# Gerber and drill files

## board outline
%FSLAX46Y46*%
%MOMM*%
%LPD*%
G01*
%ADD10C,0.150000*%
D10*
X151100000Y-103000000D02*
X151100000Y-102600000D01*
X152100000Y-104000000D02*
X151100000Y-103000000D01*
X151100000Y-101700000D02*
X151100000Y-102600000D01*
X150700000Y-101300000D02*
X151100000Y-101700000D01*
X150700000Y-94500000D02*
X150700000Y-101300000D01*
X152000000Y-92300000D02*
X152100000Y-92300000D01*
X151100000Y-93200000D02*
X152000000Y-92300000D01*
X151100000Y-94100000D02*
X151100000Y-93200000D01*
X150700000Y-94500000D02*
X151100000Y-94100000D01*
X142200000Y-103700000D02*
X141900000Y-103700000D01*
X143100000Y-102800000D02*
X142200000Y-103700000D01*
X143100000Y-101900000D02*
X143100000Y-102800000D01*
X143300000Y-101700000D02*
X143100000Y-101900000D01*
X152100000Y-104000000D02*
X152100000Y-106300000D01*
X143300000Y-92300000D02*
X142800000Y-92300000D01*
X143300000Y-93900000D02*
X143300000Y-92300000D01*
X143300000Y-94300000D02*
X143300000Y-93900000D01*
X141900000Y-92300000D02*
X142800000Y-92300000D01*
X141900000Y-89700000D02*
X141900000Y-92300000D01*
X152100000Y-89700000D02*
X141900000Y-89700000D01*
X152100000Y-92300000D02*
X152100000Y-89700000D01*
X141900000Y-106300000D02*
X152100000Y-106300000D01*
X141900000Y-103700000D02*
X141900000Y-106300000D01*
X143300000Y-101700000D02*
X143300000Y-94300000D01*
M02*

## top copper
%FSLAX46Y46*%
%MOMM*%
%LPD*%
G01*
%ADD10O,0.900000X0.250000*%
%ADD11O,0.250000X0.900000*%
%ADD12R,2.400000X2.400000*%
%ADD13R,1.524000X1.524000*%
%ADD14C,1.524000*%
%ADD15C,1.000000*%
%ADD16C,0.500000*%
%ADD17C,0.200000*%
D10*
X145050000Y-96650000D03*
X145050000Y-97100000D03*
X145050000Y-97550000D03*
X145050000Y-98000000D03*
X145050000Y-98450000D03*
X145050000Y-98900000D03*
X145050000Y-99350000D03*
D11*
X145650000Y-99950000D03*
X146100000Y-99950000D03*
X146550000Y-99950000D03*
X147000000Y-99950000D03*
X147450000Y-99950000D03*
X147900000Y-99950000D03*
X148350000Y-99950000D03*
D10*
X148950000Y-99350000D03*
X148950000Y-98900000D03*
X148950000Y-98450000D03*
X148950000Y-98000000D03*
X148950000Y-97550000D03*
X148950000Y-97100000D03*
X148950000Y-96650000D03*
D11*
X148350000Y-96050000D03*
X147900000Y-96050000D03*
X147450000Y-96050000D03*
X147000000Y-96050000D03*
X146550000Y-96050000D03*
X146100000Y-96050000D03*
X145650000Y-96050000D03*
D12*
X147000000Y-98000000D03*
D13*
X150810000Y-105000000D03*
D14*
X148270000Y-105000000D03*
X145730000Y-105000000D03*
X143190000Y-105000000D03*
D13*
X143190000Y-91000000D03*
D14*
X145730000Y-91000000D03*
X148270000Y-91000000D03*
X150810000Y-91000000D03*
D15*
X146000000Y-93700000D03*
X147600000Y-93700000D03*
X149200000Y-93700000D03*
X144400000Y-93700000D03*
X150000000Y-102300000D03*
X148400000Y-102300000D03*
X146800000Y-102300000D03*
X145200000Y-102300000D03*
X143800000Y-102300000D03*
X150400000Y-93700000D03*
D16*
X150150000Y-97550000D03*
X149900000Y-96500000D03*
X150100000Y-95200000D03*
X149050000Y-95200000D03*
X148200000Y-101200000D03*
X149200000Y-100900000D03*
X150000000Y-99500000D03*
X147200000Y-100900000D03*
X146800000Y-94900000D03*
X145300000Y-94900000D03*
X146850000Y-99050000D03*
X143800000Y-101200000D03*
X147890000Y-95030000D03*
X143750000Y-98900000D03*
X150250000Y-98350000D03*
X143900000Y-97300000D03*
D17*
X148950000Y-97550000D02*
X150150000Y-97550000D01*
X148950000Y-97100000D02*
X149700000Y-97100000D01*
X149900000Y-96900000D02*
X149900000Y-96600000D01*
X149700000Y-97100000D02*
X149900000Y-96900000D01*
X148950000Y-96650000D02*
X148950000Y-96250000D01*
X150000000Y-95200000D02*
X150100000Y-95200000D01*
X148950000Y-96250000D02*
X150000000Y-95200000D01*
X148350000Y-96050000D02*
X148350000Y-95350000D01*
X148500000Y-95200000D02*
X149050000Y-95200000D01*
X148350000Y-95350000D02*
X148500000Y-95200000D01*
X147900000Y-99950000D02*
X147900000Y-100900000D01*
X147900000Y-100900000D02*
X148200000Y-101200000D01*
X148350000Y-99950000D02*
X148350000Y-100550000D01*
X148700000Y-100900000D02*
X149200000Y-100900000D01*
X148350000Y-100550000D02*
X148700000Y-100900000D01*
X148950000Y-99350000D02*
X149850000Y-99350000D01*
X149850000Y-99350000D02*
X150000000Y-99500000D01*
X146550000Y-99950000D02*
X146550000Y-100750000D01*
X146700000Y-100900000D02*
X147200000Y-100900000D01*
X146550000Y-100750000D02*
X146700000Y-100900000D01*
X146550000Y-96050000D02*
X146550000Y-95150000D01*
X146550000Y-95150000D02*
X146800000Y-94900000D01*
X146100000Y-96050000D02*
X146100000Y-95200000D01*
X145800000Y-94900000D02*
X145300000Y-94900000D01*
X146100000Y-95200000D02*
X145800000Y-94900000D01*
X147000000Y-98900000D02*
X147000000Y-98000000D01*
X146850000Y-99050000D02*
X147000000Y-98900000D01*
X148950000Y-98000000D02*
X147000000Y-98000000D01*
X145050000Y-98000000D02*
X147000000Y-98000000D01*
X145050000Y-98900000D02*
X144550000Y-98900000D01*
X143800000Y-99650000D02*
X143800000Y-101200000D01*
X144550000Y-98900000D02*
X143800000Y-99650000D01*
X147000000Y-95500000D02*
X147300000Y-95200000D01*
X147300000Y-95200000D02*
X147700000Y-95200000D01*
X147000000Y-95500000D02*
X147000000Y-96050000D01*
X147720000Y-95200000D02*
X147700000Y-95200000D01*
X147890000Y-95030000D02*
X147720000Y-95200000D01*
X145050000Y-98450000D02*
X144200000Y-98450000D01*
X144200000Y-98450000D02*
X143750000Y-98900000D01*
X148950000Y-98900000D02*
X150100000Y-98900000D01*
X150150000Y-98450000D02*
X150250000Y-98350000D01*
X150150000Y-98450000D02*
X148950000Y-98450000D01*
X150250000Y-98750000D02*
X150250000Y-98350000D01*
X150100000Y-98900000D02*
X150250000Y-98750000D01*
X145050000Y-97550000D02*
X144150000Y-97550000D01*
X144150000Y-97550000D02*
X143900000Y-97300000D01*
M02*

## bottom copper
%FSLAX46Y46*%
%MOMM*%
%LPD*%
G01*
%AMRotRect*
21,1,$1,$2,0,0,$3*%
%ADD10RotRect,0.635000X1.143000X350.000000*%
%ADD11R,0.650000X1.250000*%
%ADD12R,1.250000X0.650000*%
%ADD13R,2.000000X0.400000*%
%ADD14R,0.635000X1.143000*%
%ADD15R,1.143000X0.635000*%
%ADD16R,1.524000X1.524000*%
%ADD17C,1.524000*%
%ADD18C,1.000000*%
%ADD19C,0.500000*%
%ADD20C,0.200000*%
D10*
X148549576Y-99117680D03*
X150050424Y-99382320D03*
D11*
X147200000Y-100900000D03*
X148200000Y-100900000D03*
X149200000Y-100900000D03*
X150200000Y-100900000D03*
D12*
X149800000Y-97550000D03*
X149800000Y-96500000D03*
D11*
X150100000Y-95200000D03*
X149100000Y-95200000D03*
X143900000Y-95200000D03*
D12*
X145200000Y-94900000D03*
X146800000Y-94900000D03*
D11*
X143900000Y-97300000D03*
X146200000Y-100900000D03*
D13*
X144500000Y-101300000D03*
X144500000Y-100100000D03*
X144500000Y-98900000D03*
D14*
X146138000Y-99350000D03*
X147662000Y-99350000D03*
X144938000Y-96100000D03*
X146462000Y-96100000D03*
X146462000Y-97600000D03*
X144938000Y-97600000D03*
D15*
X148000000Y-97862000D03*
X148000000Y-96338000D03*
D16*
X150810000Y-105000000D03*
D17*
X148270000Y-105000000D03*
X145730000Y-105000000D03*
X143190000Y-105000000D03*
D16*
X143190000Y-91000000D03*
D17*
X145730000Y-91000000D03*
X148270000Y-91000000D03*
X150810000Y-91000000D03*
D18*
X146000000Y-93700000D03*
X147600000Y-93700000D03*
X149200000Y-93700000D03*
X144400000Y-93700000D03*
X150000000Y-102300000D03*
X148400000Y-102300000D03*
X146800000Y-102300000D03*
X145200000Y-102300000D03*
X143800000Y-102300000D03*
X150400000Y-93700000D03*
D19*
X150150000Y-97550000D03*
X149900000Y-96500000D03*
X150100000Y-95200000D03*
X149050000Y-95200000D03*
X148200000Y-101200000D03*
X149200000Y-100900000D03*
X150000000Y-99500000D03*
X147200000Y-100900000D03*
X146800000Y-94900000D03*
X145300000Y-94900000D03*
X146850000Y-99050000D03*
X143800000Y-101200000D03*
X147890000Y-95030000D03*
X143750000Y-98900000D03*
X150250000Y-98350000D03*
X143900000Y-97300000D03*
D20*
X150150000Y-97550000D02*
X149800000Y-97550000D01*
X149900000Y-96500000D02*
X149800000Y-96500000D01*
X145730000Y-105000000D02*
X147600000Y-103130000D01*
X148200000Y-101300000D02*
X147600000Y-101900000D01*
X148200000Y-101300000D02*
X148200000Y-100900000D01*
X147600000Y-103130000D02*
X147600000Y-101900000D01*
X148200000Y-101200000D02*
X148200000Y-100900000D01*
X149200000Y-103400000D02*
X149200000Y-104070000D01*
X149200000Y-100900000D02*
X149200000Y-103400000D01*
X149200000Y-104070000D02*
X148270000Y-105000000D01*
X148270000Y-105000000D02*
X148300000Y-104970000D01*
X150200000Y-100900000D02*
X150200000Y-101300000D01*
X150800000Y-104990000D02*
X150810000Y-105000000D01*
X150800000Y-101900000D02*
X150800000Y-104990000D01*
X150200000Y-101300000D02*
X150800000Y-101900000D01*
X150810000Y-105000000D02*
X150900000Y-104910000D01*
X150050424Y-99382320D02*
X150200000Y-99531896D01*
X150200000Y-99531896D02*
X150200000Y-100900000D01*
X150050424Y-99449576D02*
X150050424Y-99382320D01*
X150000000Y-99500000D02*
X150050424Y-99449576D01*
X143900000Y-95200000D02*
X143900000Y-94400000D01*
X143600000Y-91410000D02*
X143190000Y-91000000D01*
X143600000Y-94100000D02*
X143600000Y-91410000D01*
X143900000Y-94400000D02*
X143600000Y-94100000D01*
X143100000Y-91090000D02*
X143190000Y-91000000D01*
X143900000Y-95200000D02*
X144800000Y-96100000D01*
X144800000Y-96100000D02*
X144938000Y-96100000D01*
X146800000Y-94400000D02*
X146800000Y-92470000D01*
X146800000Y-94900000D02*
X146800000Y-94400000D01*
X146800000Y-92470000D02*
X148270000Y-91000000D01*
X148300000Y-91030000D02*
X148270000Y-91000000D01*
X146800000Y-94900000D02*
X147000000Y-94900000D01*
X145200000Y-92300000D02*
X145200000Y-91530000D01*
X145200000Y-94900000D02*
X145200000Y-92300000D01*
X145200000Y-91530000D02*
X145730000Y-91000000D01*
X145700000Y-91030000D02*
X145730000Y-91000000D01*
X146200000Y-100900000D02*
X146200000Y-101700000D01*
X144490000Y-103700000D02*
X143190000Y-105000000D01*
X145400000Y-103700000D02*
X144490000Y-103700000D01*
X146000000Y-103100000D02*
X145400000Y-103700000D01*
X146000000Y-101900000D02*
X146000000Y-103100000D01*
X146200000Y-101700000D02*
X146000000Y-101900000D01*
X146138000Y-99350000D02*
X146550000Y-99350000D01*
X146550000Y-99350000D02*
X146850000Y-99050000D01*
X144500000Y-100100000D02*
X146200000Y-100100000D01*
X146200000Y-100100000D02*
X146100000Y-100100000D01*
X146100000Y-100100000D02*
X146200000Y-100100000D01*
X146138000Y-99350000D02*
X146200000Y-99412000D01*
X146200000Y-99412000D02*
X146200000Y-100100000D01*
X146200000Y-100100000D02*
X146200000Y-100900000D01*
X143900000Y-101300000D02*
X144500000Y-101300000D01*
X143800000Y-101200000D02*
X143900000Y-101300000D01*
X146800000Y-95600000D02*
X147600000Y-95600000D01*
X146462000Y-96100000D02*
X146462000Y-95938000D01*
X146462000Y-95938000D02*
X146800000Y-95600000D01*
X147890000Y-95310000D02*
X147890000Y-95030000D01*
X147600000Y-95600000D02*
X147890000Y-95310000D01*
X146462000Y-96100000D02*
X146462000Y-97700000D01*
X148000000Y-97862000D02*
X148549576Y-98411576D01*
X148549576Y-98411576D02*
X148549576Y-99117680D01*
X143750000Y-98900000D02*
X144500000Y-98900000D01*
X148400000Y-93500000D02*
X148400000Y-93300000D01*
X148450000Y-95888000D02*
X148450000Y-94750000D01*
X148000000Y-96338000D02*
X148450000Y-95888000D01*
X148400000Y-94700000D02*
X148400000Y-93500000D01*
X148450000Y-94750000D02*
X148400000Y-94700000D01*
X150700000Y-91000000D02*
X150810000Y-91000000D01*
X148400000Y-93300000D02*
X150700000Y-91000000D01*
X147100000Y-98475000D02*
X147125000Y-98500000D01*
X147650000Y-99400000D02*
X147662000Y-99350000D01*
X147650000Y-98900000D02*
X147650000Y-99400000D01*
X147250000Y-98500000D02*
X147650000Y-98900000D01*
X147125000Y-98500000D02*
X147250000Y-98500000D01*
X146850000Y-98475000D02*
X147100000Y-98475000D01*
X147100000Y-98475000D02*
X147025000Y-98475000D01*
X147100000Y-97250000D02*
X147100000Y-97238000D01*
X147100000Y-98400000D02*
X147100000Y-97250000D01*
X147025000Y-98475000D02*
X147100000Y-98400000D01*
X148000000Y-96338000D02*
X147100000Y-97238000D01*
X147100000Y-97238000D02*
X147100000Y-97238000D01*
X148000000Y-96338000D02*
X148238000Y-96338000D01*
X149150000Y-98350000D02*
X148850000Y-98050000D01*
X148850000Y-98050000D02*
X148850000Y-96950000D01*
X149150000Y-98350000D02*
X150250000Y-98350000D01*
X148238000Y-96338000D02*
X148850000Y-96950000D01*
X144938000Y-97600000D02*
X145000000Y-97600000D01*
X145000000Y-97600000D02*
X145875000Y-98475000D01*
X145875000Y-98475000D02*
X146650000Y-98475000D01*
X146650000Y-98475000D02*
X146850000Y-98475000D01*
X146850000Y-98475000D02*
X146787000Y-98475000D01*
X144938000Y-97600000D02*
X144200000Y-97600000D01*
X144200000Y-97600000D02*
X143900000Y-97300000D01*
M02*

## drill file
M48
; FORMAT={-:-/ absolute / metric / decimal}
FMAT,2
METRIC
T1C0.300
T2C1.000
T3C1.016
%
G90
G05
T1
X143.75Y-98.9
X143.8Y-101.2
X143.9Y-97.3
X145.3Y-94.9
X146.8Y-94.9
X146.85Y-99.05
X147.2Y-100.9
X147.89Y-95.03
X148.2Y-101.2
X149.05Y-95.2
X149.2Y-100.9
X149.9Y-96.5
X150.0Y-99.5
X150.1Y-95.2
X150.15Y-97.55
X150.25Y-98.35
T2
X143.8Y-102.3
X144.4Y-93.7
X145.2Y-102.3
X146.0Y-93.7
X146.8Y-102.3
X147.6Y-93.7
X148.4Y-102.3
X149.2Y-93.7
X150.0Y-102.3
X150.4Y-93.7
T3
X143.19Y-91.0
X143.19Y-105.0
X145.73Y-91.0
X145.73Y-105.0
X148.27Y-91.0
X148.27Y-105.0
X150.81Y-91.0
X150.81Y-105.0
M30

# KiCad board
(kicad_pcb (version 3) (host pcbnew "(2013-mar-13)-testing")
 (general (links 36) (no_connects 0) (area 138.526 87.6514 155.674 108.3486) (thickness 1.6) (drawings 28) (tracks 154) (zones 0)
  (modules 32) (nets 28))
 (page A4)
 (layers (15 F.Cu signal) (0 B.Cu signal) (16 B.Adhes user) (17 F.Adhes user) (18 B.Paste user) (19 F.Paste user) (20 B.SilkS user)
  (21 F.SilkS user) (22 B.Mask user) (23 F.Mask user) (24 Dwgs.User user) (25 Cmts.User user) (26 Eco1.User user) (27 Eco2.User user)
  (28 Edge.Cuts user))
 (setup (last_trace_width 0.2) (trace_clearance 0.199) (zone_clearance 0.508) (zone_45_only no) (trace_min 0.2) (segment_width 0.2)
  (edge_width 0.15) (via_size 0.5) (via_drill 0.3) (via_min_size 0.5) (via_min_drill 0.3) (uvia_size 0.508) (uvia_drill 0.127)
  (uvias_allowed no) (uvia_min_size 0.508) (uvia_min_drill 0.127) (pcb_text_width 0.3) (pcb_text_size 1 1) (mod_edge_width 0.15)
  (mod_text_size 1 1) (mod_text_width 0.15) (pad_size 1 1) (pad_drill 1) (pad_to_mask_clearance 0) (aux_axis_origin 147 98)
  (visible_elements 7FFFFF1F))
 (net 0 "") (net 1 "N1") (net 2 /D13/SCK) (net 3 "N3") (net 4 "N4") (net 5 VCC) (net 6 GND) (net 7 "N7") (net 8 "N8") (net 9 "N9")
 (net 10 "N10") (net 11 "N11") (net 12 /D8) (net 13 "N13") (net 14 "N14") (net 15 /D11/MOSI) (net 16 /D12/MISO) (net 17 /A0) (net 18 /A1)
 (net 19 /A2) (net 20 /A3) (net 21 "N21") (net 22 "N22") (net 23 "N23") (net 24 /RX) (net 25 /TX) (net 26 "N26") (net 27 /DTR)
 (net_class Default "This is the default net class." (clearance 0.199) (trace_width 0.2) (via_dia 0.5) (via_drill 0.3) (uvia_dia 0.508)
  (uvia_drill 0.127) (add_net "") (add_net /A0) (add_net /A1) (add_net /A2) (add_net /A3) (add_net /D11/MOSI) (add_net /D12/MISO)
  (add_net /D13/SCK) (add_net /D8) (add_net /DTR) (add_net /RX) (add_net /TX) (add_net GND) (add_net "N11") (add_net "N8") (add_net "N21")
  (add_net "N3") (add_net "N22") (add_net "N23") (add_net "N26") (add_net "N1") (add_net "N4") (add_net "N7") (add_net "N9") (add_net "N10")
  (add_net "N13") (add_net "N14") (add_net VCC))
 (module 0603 (layer B.Cu) (at 149.3 99.25 350)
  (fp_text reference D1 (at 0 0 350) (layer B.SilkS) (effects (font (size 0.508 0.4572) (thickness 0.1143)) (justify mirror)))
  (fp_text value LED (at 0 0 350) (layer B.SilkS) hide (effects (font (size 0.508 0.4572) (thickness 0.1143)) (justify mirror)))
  (pad 1 smd rect (at -0.762 0 350) (size 0.635 1.143) (layers B.Cu B.Paste B.Mask) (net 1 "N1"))
  (pad 2 smd rect (at 0.762 0 350) (size 0.635 1.143) (layers B.Cu B.Paste B.Mask) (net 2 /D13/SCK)))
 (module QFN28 (layer F.Cu) (at 147 98)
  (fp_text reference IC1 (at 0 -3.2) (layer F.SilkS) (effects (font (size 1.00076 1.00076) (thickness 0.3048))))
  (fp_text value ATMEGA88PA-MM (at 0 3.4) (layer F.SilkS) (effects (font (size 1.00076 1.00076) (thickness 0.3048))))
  (pad 1 smd oval (at -1.95 -1.35) (size 0.9 0.25) (layers F.Cu F.Paste F.Mask) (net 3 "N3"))
  (pad 2 smd oval (at -1.95 -0.9) (size 0.9 0.25) (layers F.Cu F.Paste F.Mask) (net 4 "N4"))
  (pad 3 smd oval (at -1.95 -0.45) (size 0.9 0.25) (layers F.Cu F.Paste F.Mask) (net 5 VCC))
  (pad 4 smd oval (at -1.95 0) (size 0.9 0.25) (layers F.Cu F.Paste F.Mask) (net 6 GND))
  (pad 5 smd oval (at -1.95 0.45) (size 0.9 0.25) (layers F.Cu F.Paste F.Mask) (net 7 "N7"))
  (pad 6 smd oval (at -1.95 0.9) (size 0.9 0.25) (layers F.Cu F.Paste F.Mask) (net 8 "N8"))
  (pad 7 smd oval (at -1.95 1.35) (size 0.9 0.25) (layers F.Cu F.Paste F.Mask) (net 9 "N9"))
  (pad 8 smd oval (at -1.35 1.95 90) (size 0.9 0.25) (layers F.Cu F.Paste F.Mask) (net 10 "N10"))
  (pad 9 smd oval (at -0.9 1.95 90) (size 0.9 0.25) (layers F.Cu F.Paste F.Mask) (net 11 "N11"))
  (pad 10 smd oval (at -0.45 1.95 90) (size 0.9 0.25) (layers F.Cu F.Paste F.Mask) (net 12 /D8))
  (pad 11 smd oval (at 0 1.95 90) (size 0.9 0.25) (layers F.Cu F.Paste F.Mask) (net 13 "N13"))
  (pad 12 smd oval (at 0.45 1.95 90) (size 0.9 0.25) (layers F.Cu F.Paste F.Mask) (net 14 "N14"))
  (pad 13 smd oval (at 0.9 1.95 90) (size 0.9 0.25) (layers F.Cu F.Paste F.Mask) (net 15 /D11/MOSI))
  (pad 14 smd oval (at 1.35 1.95 90) (size 0.9 0.25) (layers F.Cu F.Paste F.Mask) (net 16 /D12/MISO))
  (pad 15 smd oval (at 1.95 1.35) (size 0.9 0.25) (layers F.Cu F.Paste F.Mask) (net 2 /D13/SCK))
  (pad 16 smd oval (at 1.95 0.9) (size 0.9 0.25) (layers F.Cu F.Paste F.Mask) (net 5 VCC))
  (pad 17 smd oval (at 1.95 0.45) (size 0.9 0.25) (layers F.Cu F.Paste F.Mask) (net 5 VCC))
  (pad 18 smd oval (at 1.95 0) (size 0.9 0.25) (layers F.Cu F.Paste F.Mask) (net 6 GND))
  (pad 19 smd oval (at 1.95 -0.45) (size 0.9 0.25) (layers F.Cu F.Paste F.Mask) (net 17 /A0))
  (pad 20 smd oval (at 1.95 -0.9) (size 0.9 0.25) (layers F.Cu F.Paste F.Mask) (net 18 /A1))
  (pad 21 smd oval (at 1.95 -1.35) (size 0.9 0.25) (layers F.Cu F.Paste F.Mask) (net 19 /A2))
  (pad 22 smd oval (at 1.35 -1.95 90) (size 0.9 0.25) (layers F.Cu F.Paste F.Mask) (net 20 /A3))
  (pad 23 smd oval (at 0.9 -1.95 90) (size 0.9 0.25) (layers F.Cu F.Paste F.Mask) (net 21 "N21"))
  (pad 24 smd oval (at 0.45 -1.95 90) (size 0.9 0.25) (layers F.Cu F.Paste F.Mask) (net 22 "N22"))
  (pad 25 smd oval (at 0 -1.95 90) (size 0.9 0.25) (layers F.Cu F.Paste F.Mask) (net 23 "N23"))
  (pad 26 smd oval (at -0.45 -1.95 90) (size 0.9 0.25) (layers F.Cu F.Paste F.Mask) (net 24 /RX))
  (pad 27 smd oval (at -0.9 -1.95 90) (size 0.9 0.25) (layers F.Cu F.Paste F.Mask) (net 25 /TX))
  (pad 28 smd oval (at -1.35 -1.95 90) (size 0.9 0.25) (layers F.Cu F.Paste F.Mask) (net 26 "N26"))
  (pad 0 smd rect (at 0 0) (size 2.4 2.4) (layers F.Cu F.Paste F.Mask) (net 6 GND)))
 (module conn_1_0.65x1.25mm (layer B.Cu) (at 147.2 100.9 270)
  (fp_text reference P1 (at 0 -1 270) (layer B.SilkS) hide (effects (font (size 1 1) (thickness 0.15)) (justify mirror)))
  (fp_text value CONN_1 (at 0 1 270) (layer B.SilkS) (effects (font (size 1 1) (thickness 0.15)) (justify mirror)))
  (pad 1 smd rect (at 0 0 270) (size 1.25 0.65) (layers B.Cu B.Mask) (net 12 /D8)))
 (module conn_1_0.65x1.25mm (layer B.Cu) (at 148.2 100.9 90)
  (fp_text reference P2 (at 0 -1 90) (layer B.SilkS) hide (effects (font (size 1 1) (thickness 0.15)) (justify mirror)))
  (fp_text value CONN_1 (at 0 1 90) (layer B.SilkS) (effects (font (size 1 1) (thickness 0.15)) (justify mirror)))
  (pad 1 smd rect (at 0 0 90) (size 1.25 0.65) (layers B.Cu B.Mask) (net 15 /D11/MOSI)))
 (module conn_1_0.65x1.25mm (layer B.Cu) (at 149.2 100.9 270)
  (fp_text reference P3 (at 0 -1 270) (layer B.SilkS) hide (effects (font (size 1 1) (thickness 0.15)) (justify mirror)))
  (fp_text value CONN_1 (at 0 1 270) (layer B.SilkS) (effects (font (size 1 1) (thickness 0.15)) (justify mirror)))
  (pad 1 smd rect (at 0 0 270) (size 1.25 0.65) (layers B.Cu B.Mask) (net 16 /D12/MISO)))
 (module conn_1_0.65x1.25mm (layer B.Cu) (at 150.2 100.9 270)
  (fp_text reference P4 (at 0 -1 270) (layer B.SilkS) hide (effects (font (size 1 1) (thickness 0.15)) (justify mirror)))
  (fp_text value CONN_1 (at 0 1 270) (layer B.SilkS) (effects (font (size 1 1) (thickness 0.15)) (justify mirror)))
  (pad 1 smd rect (at 0 0 270) (size 1.25 0.65) (layers B.Cu B.Mask) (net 2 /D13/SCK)))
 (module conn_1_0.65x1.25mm (layer B.Cu) (at 149.8 97.55)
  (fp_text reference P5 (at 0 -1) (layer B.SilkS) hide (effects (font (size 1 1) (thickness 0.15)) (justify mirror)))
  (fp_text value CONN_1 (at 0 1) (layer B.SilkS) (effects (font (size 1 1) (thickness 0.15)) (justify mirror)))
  (pad 1 smd rect (at 0 0) (size 1.25 0.65) (layers B.Cu B.Mask) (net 17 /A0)))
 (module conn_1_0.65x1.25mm (layer B.Cu) (at 149.8 96.5)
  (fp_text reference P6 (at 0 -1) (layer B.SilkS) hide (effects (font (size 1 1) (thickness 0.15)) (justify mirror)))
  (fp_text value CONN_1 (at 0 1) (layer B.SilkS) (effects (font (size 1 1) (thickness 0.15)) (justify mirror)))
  (pad 1 smd rect (at 0 0) (size 1.25 0.65) (layers B.Cu B.Mask) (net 18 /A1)))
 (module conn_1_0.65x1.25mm (layer B.Cu) (at 150.1 95.2 90)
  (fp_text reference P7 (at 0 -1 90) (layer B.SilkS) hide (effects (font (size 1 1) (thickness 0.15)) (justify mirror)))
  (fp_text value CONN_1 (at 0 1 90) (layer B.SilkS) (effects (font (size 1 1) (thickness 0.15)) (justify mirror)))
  (pad 1 smd rect (at 0 0 90) (size 1.25 0.65) (layers B.Cu B.Mask) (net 19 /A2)))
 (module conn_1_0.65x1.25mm (layer B.Cu) (at 149.1 95.2 90)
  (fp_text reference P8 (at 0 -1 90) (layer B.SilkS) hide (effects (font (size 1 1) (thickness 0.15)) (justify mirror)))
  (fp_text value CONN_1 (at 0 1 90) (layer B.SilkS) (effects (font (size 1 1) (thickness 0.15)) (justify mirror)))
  (pad 1 smd rect (at 0 0 90) (size 1.25 0.65) (layers B.Cu B.Mask) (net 20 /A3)))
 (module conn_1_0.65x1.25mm (layer B.Cu) (at 143.9 95.2 90)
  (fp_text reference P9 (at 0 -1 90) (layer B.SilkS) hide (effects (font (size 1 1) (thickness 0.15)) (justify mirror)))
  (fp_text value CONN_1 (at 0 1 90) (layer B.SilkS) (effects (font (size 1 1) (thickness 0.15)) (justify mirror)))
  (pad 1 smd rect (at 0 0 90) (size 1.25 0.65) (layers B.Cu B.Mask) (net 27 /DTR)))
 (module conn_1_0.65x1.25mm (layer B.Cu) (at 145.2 94.9)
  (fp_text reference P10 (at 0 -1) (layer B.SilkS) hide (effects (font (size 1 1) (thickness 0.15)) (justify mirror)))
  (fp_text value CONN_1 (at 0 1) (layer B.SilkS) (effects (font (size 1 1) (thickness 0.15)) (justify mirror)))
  (pad 1 smd rect (at 0 0) (size 1.25 0.65) (layers B.Cu B.Mask) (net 25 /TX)))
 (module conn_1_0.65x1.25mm (layer B.Cu) (at 146.8 94.9)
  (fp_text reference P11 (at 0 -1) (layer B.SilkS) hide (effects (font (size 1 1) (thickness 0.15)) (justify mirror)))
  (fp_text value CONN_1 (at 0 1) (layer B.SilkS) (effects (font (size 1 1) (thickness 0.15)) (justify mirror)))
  (pad 1 smd rect (at 0 0) (size 1.25 0.65) (layers B.Cu B.Mask) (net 24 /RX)))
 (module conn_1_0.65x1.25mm (layer B.Cu) (at 143.9 97.3 90)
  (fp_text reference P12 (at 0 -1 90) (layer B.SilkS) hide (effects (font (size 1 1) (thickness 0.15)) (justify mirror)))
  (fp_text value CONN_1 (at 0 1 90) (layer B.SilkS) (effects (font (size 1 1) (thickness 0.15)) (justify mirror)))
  (pad 1 smd rect (at 0 0 90) (size 1.25 0.65) (layers B.Cu B.Mask) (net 5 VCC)))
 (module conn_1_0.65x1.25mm (layer B.Cu) (at 146.2 100.9 90)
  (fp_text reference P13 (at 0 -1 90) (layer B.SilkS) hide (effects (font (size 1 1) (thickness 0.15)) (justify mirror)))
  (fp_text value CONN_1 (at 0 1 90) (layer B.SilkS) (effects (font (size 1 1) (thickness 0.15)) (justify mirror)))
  (pad 1 smd rect (at 0 0 90) (size 1.25 0.65) (layers B.Cu B.Mask) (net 6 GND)))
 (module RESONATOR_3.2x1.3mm (layer B.Cu) (at 144.5 100.1 90)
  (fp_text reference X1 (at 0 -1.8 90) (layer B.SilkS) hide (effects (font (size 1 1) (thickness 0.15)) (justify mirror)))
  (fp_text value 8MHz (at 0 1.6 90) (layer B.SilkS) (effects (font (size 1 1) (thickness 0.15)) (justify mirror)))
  (pad 1 smd rect (at -1.2 0 90) (size 0.4 2) (layers B.Cu B.Mask) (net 8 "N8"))
  (pad 2 smd rect (at 0 0 90) (size 0.4 2) (layers B.Cu B.Mask) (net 6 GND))
  (pad 3 smd rect (at 1.2 0 90) (size 0.4 2) (layers B.Cu B.Mask) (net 7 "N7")))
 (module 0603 (layer B.Cu) (at 146.9 99.35)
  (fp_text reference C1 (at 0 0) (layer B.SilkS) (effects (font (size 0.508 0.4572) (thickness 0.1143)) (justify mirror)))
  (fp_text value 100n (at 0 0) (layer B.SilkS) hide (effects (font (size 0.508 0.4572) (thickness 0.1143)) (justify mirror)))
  (pad 1 smd rect (at -0.762 0) (size 0.635 1.143) (layers B.Cu B.Paste B.Mask) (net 6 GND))
  (pad 2 smd rect (at 0.762 0) (size 0.635 1.143) (layers B.Cu B.Paste B.Mask) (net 5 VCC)))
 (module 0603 (layer B.Cu) (at 145.7 96.1)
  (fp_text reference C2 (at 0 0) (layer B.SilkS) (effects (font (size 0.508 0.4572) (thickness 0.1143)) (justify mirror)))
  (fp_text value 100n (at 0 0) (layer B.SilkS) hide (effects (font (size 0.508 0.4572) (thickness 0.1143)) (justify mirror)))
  (pad 1 smd rect (at -0.762 0) (size 0.635 1.143) (layers B.Cu B.Paste B.Mask) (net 27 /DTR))
  (pad 2 smd rect (at 0.762 0) (size 0.635 1.143) (layers B.Cu B.Paste B.Mask) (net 23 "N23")))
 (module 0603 (layer B.Cu) (at 145.7 97.6 180)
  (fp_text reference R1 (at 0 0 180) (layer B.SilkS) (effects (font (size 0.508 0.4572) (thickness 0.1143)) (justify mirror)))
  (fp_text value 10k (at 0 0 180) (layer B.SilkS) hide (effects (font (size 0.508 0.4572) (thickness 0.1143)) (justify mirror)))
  (pad 1 smd rect (at -0.762 0 180) (size 0.635 1.143) (layers B.Cu B.Paste B.Mask) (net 23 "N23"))
  (pad 2 smd rect (at 0.762 0 180) (size 0.635 1.143) (layers B.Cu B.Paste B.Mask) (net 5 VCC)))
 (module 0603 (layer B.Cu) (at 148 97.1 90)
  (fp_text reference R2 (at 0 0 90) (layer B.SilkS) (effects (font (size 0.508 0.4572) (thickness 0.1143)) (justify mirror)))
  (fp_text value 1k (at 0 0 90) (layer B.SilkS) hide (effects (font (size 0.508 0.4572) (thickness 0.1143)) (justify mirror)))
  (pad 1 smd rect (at -0.762 0 90) (size 0.635 1.143) (layers B.Cu B.Paste B.Mask) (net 1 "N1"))
  (pad 2 smd rect (at 0.762 0 90) (size 0.635 1.143) (layers B.Cu B.Paste B.Mask) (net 5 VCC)))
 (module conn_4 (layer F.Cu) (at 147 105 180)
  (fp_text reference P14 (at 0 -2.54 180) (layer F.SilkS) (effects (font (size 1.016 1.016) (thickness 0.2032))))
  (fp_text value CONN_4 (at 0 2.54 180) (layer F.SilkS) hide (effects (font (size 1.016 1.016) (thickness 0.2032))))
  (pad 1 thru_hole rect (at -3.81 0 180) (size 1.524 1.524) (drill 1.016) (layers *.Cu *.Mask F.SilkS) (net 2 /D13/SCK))
  (pad 2 thru_hole circle (at -1.27 0 180) (size 1.524 1.524) (drill 1.016) (layers *.Cu *.Mask F.SilkS) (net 16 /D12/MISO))
  (pad 3 thru_hole circle (at 1.27 0 180) (size 1.524 1.524) (drill 1.016) (layers *.Cu *.Mask F.SilkS) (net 15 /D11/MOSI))
  (pad 4 thru_hole circle (at 3.81 0 180) (size 1.524 1.524) (drill 1.016) (layers *.Cu *.Mask F.SilkS) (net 6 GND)))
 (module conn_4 (layer F.Cu) (at 147 91)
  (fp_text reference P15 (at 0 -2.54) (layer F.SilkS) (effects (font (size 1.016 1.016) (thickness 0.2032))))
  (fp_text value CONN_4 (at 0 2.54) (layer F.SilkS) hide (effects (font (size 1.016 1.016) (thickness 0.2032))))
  (pad 1 thru_hole rect (at -3.81 0) (size 1.524 1.524) (drill 1.016) (layers *.Cu *.Mask F.SilkS) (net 27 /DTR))
  (pad 2 thru_hole circle (at -1.27 0) (size 1.524 1.524) (drill 1.016) (layers *.Cu *.Mask F.SilkS) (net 25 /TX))
  (pad 3 thru_hole circle (at 1.27 0) (size 1.524 1.524) (drill 1.016) (layers *.Cu *.Mask F.SilkS) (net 24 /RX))
  (pad 4 thru_hole circle (at 3.81 0) (size 1.524 1.524) (drill 1.016) (layers *.Cu *.Mask F.SilkS) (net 5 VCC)))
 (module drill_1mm (layer F.Cu) (at 146 93.7)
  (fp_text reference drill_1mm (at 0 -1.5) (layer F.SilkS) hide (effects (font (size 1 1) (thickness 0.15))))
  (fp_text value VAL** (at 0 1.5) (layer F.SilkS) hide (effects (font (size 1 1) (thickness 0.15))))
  (pad "" thru_hole circle (at 0 0) (size 1 1) (drill 1) (layers *.Cu)))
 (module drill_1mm (layer F.Cu) (at 147.6 93.7)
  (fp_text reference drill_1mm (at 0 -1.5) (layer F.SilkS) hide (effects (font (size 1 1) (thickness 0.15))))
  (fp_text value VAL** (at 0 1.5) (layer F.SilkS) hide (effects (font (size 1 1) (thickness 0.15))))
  (pad "" thru_hole circle (at 0 0) (size 1 1) (drill 1) (layers *.Cu)))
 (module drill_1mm (layer F.Cu) (at 149.2 93.7)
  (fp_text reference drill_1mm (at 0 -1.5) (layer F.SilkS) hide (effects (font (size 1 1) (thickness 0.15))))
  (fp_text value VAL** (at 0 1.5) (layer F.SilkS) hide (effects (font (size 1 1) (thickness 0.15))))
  (pad "" thru_hole circle (at 0 0) (size 1 1) (drill 1) (layers *.Cu)))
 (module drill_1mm (layer F.Cu) (at 144.4 93.7)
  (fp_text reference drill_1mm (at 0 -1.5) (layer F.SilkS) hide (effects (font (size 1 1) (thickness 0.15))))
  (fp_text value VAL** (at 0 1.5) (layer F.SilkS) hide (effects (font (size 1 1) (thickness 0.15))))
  (pad "" thru_hole circle (at 0 0) (size 1 1) (drill 1) (layers *.Cu)))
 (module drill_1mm (layer F.Cu) (at 150 102.3)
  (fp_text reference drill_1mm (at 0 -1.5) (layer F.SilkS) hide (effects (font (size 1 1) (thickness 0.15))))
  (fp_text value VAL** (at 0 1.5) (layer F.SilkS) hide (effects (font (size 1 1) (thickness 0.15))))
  (pad "" thru_hole circle (at 0 0) (size 1 1) (drill 1) (layers *.Cu)))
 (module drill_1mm (layer F.Cu) (at 148.4 102.3)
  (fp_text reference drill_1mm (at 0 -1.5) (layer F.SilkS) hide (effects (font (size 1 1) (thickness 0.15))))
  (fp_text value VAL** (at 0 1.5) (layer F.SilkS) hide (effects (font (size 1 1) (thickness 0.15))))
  (pad "" thru_hole circle (at 0 0) (size 1 1) (drill 1) (layers *.Cu)))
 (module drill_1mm (layer F.Cu) (at 146.8 102.3)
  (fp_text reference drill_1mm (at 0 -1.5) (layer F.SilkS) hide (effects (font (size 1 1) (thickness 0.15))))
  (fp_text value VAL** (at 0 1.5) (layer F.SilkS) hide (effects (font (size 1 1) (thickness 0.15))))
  (pad "" thru_hole circle (at 0 0) (size 1 1) (drill 1) (layers *.Cu)))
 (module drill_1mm (layer F.Cu) (at 145.2 102.3)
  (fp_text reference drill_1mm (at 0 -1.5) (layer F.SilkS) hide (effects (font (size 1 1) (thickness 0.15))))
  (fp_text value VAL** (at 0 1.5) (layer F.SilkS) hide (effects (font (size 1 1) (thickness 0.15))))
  (pad "" thru_hole circle (at 0 0) (size 1 1) (drill 1) (layers *.Cu)))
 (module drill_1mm (layer F.Cu) (at 143.8 102.3)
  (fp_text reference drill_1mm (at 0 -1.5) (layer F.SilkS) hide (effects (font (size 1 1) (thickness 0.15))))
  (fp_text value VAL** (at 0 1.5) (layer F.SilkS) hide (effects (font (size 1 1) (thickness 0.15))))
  (pad "" thru_hole circle (at 0 0) (size 1 1) (drill 1) (layers *.Cu)))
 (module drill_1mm (layer F.Cu) (at 150.4 93.7)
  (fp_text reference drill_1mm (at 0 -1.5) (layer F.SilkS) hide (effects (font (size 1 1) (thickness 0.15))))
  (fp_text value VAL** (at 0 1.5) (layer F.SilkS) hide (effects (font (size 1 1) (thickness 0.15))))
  (pad "" thru_hole circle (at 0 0) (size 1 1) (drill 1) (layers *.Cu)))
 (gr_line (start 151.1 103) (end 151.1 102.6) (angle 90) (layer Edge.Cuts) (width 0.15))
 (gr_line (start 152.1 104) (end 151.1 103) (angle 90) (layer Edge.Cuts) (width 0.15))
 (gr_line (start 151.1 101.7) (end 151.1 102.6) (angle 90) (layer Edge.Cuts) (width 0.15))
 (gr_line (start 150.7 101.3) (end 151.1 101.7) (angle 90) (layer Edge.Cuts) (width 0.15))
 (gr_line (start 150.7 94.5) (end 150.7 101.3) (angle 90) (layer Edge.Cuts) (width 0.15))
 (gr_line (start 152 92.3) (end 152.1 92.3) (angle 90) (layer Edge.Cuts) (width 0.15))
 (gr_line (start 151.1 93.2) (end 152 92.3) (angle 90) (layer Edge.Cuts) (width 0.15))
 (gr_line (start 151.1 94.1) (end 151.1 93.2) (angle 90) (layer Edge.Cuts) (width 0.15))
 (gr_line (start 150.7 94.5) (end 151.1 94.1) (angle 90) (layer Edge.Cuts) (width 0.15))
 (gr_line (start 142.2 103.7) (end 141.9 103.7) (angle 90) (layer Edge.Cuts) (width 0.15))
 (gr_line (start 143.1 102.8) (end 142.2 103.7) (angle 90) (layer Edge.Cuts) (width 0.15))
 (gr_line (start 143.1 101.9) (end 143.1 102.8) (angle 90) (layer Edge.Cuts) (width 0.15))
 (gr_line (start 143.3 101.7) (end 143.1 101.9) (angle 90) (layer Edge.Cuts) (width 0.15))
 (gr_line (start 152.1 104) (end 152.1 106.3) (angle 90) (layer Edge.Cuts) (width 0.15))
 (gr_line (start 143.3 92.3) (end 142.8 92.3) (angle 90) (layer Edge.Cuts) (width 0.15))
 (gr_line (start 143.3 93.9) (end 143.3 92.3) (angle 90) (layer Edge.Cuts) (width 0.15))
 (gr_line (start 143.3 94.3) (end 143.3 93.9) (angle 90) (layer Edge.Cuts) (width 0.15))
 (gr_line (start 141.9 92.3) (end 142.8 92.3) (angle 90) (layer Edge.Cuts) (width 0.15))
 (gr_line (start 141.9 89.7) (end 141.9 92.3) (angle 90) (layer Edge.Cuts) (width 0.15))
 (gr_line (start 152.1 89.7) (end 141.9 89.7) (angle 90) (layer Edge.Cuts) (width 0.15))
 (gr_line (start 152.1 92.3) (end 152.1 89.7) (angle 90) (layer Edge.Cuts) (width 0.15))
 (gr_line (start 141.9 106.3) (end 152.1 106.3) (angle 90) (layer Edge.Cuts) (width 0.15))
 (gr_line (start 141.9 103.7) (end 141.9 106.3) (angle 90) (layer Edge.Cuts) (width 0.15))
 (gr_line (start 143.3 101.7) (end 143.3 94.3) (angle 90) (layer Edge.Cuts) (width 0.15))
 (segment (start 148.95 97.55) (end 150.15 97.55) (width 0.2) (layer F.Cu) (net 17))
 (segment (start 150.15 97.55) (end 149.8 97.55) (width 0.2) (layer B.Cu) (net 17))
 (via (at 150.15 97.55) (size 0.5) (layers F.Cu B.Cu) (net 17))
 (segment (start 148.95 97.1) (end 149.7 97.1) (width 0.2) (layer F.Cu) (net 18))
 (segment (start 149.9 96.5) (end 149.8 96.5) (width 0.2) (layer B.Cu) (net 18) (status 30))
 (via (at 149.9 96.5) (size 0.5) (layers F.Cu B.Cu) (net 18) (status 30))
 (segment (start 149.9 96.9) (end 149.9 96.6) (width 0.2) (layer F.Cu) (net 18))
 (segment (start 149.7 97.1) (end 149.9 96.9) (width 0.2) (layer F.Cu) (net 18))
 (segment (start 148.95 96.65) (end 148.95 96.25) (width 0.2) (layer F.Cu) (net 19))
 (via (at 150.1 95.2) (size 0.5) (layers F.Cu B.Cu) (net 19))
 (segment (start 150 95.2) (end 150.1 95.2) (width 0.2) (layer F.Cu) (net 19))
 (segment (start 148.95 96.25) (end 150 95.2) (width 0.2) (layer F.Cu) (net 19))
 (segment (start 148.35 96.05) (end 148.35 95.35) (width 0.2) (layer F.Cu) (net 20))
 (via (at 149.05 95.2) (size 0.5) (layers F.Cu B.Cu) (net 20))
 (segment (start 148.5 95.2) (end 149.05 95.2) (width 0.2) (layer F.Cu) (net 20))
 (segment (start 148.35 95.35) (end 148.5 95.2) (width 0.2) (layer F.Cu) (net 20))
 (segment (start 145.73 105) (end 147.6 103.13) (width 0.2) (layer B.Cu) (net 15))
 (segment (start 148.2 101.3) (end 147.6 101.9) (width 0.2) (layer B.Cu) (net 15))
 (segment (start 148.2 101.3) (end 148.2 100.9) (width 0.2) (layer B.Cu) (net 15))
 (segment (start 147.6 103.13) (end 147.6 101.9) (width 0.2) (layer B.Cu) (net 15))
 (segment (start 147.9 99.95) (end 147.9 100.9) (width 0.2) (layer F.Cu) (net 15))
 (segment (start 148.2 101.2) (end 148.2 100.9) (width 0.2) (layer B.Cu) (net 15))
 (via (at 148.2 101.2) (size 0.5) (layers F.Cu B.Cu) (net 15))
 (segment (start 147.9 100.9) (end 148.2 101.2) (width 0.2) (layer F.Cu) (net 15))
 (segment (start 149.2 103.4) (end 149.2 104.07) (width 0.2) (layer B.Cu) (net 16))
 (segment (start 149.2 100.9) (end 149.2 103.4) (width 0.2) (layer B.Cu) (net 16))
 (segment (start 149.2 104.07) (end 148.27 105) (width 0.2) (layer B.Cu) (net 16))
 (segment (start 148.27 105) (end 148.3 104.97) (width 0.2) (layer B.Cu) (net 16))
 (segment (start 148.35 99.95) (end 148.35 100.55) (width 0.2) (layer F.Cu) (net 16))
 (via (at 149.2 100.9) (size 0.5) (layers F.Cu B.Cu) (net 16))
 (segment (start 148.7 100.9) (end 149.2 100.9) (width 0.2) (layer F.Cu) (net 16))
 (segment (start 148.35 100.55) (end 148.7 100.9) (width 0.2) (layer F.Cu) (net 16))
 (segment (start 150.2 100.9) (end 150.2 101.3) (width 0.2) (layer B.Cu) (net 2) (status C00000))
 (segment (start 150.8 104.99) (end 150.81 105) (width 0.2) (layer B.Cu) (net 2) (status C00000))
 (segment (start 150.8 101.9) (end 150.8 104.99) (width 0.2) (layer B.Cu) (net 2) (status 800000))
 (segment (start 150.2 101.3) (end 150.8 101.9) (width 0.2) (layer B.Cu) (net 2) (status 400000))
 (segment (start 150.81 105) (end 150.9 104.91) (width 0.2) (layer B.Cu) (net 2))
 (segment (start 150.050424 99.38232) (end 150.2 99.531896) (width 0.2) (layer B.Cu) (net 2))
 (segment (start 150.2 99.531896) (end 150.2 100.9) (width 0.2) (layer B.Cu) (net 2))
 (segment (start 148.95 99.35) (end 149.85 99.35) (width 0.2) (layer F.Cu) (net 2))
 (segment (start 150.050424 99.449576) (end 150.050424 99.38232) (width 0.2) (layer B.Cu) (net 2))
 (segment (start 150 99.5) (end 150.050424 99.449576) (width 0.2) (layer B.Cu) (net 2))
 (via (at 150 99.5) (size 0.5) (layers F.Cu B.Cu) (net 2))
 (segment (start 149.85 99.35) (end 150 99.5) (width 0.2) (layer F.Cu) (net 2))
 (segment (start 146.55 99.95) (end 146.55 100.75) (width 0.2) (layer F.Cu) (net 12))
 (via (at 147.2 100.9) (size 0.5) (layers F.Cu B.Cu) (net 12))
 (segment (start 146.7 100.9) (end 147.2 100.9) (width 0.2) (layer F.Cu) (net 12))
 (segment (start 146.55 100.75) (end 146.7 100.9) (width 0.2) (layer F.Cu) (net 12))
 (segment (start 143.9 95.2) (end 143.9 94.4) (width 0.2) (layer B.Cu) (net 27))
 (segment (start 143.6 91.41) (end 143.19 91) (width 0.2) (layer B.Cu) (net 27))
 (segment (start 143.6 94.1) (end 143.6 91.41) (width 0.2) (layer B.Cu) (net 27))
 (segment (start 143.9 94.4) (end 143.6 94.1) (width 0.2) (layer B.Cu) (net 27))
 (segment (start 143.1 91.09) (end 143.19 91) (width 0.2) (layer B.Cu) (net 27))
 (segment (start 143.9 95.2) (end 144.8 96.1) (width 0.2) (layer B.Cu) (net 27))
 (segment (start 144.8 96.1) (end 144.938 96.1) (width 0.2) (layer B.Cu) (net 27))
 (segment (start 146.8 94.4) (end 146.8 92.47) (width 0.2) (layer B.Cu) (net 24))
 (segment (start 146.8 94.9) (end 146.8 94.4) (width 0.2) (layer B.Cu) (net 24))
 (segment (start 146.8 92.47) (end 148.27 91) (width 0.2) (layer B.Cu) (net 24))
 (segment (start 148.3 91.03) (end 148.27 91) (width 0.2) (layer B.Cu) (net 24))
 (segment (start 146.55 96.05) (end 146.55 95.15) (width 0.2) (layer F.Cu) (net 24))
 (segment (start 146.8 94.9) (end 147 94.9) (width 0.2) (layer B.Cu) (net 24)) (via (at 146.8 94.9) (size 0.5) (layers F.Cu B.Cu) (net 24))
 (segment (start 146.55 95.15) (end 146.8 94.9) (width 0.2) (layer F.Cu) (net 24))
 (segment (start 145.2 92.3) (end 145.2 91.53) (width 0.2) (layer B.Cu) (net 25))
 (segment (start 145.2 94.9) (end 145.2 92.3) (width 0.2) (layer B.Cu) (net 25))
 (segment (start 145.2 91.53) (end 145.73 91) (width 0.2) (layer B.Cu) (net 25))
 (segment (start 145.7 91.03) (end 145.73 91) (width 0.2) (layer B.Cu) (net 25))
 (segment (start 146.1 96.05) (end 146.1 95.2) (width 0.2) (layer F.Cu) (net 25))
 (via (at 145.3 94.9) (size 0.5) (layers F.Cu B.Cu) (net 25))
 (segment (start 145.8 94.9) (end 145.3 94.9) (width 0.2) (layer F.Cu) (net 25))
 (segment (start 146.1 95.2) (end 145.8 94.9) (width 0.2) (layer F.Cu) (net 25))
 (segment (start 146.2 100.9) (end 146.2 101.7) (width 0.2) (layer B.Cu) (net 6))
 (segment (start 144.49 103.7) (end 143.19 105) (width 0.2) (layer B.Cu) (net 6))
 (segment (start 145.4 103.7) (end 144.49 103.7) (width 0.2) (layer B.Cu) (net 6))
 (segment (start 146 103.1) (end 145.4 103.7) (width 0.2) (layer B.Cu) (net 6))
 (segment (start 146 101.9) (end 146 103.1) (width 0.2) (layer B.Cu) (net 6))
 (segment (start 146.2 101.7) (end 146 101.9) (width 0.2) (layer B.Cu) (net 6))
 (segment (start 146.138 99.35) (end 146.55 99.35) (width 0.2) (layer B.Cu) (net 6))
 (segment (start 147 98.9) (end 147 98) (width 0.2) (layer F.Cu) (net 6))
 (segment (start 146.85 99.05) (end 147 98.9) (width 0.2) (layer F.Cu) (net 6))
 (via (at 146.85 99.05) (size 0.5) (layers F.Cu B.Cu) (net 6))
 (segment (start 146.55 99.35) (end 146.85 99.05) (width 0.2) (layer B.Cu) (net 6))
 (segment (start 148.95 98) (end 147 98) (width 0.2) (layer F.Cu) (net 6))
 (segment (start 145.05 98) (end 147 98) (width 0.2) (layer F.Cu) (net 6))
 (segment (start 144.5 100.1) (end 146.2 100.1) (width 0.2) (layer B.Cu) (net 6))
 (segment (start 146.2 100.1) (end 146.1 100.1) (width 0.2) (layer B.Cu) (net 6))
 (segment (start 146.1 100.1) (end 146.2 100.1) (width 0.2) (layer B.Cu) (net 6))
 (segment (start 146.138 99.35) (end 146.2 99.412) (width 0.2) (layer B.Cu) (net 6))
 (segment (start 146.2 99.412) (end 146.2 100.1) (width 0.2) (layer B.Cu) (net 6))
 (segment (start 146.2 100.1) (end 146.2 100.9) (width 0.2) (layer B.Cu) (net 6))
 (segment (start 145.05 98.9) (end 144.55 98.9) (width 0.2) (layer F.Cu) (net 8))
 (segment (start 143.9 101.3) (end 144.5 101.3) (width 0.2) (layer B.Cu) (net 8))
 (segment (start 143.8 101.2) (end 143.9 101.3) (width 0.2) (layer B.Cu) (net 8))
 (via (at 143.8 101.2) (size 0.5) (layers F.Cu B.Cu) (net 8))
 (segment (start 143.8 99.65) (end 143.8 101.2) (width 0.2) (layer F.Cu) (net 8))
 (segment (start 144.55 98.9) (end 143.8 99.65) (width 0.2) (layer F.Cu) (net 8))
 (segment (start 146.8 95.6) (end 147.6 95.6) (width 0.2) (layer B.Cu) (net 23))
 (segment (start 147 95.5) (end 147.3 95.2) (width 0.2) (layer F.Cu) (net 23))
 (segment (start 147.3 95.2) (end 147.7 95.2) (width 0.2) (layer F.Cu) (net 23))
 (segment (start 146.462 96.1) (end 146.462 95.938) (width 0.2) (layer B.Cu) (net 23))
 (segment (start 146.462 95.938) (end 146.8 95.6) (width 0.2) (layer B.Cu) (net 23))
 (segment (start 147 95.5) (end 147 96.05) (width 0.2) (layer F.Cu) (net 23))
 (segment (start 147.72 95.2) (end 147.7 95.2) (width 0.2) (layer F.Cu) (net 23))
 (segment (start 147.89 95.03) (end 147.72 95.2) (width 0.2) (layer F.Cu) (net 23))
 (via (at 147.89 95.03) (size 0.5) (layers F.Cu B.Cu) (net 23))
 (segment (start 147.89 95.31) (end 147.89 95.03) (width 0.2) (layer B.Cu) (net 23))
 (segment (start 147.6 95.6) (end 147.89 95.31) (width 0.2) (layer B.Cu) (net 23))
 (segment (start 146.462 96.1) (end 146.462 97.7) (width 0.2) (layer B.Cu) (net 23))
 (segment (start 148 97.862) (end 148.549576 98.411576) (width 0.2) (layer B.Cu) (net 1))
 (segment (start 148.549576 98.411576) (end 148.549576 99.11768) (width 0.2) (layer B.Cu) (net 1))
 (segment (start 145.05 98.45) (end 144.2 98.45) (width 0.2) (layer F.Cu) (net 7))
 (segment (start 143.75 98.9) (end 144.5 98.9) (width 0.2) (layer B.Cu) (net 7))
 (via (at 143.75 98.9) (size 0.5) (layers F.Cu B.Cu) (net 7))
 (segment (start 144.2 98.45) (end 143.75 98.9) (width 0.2) (layer F.Cu) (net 7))
 (segment (start 148.4 93.5) (end 148.4 93.3) (width 0.2) (layer B.Cu) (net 5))
 (segment (start 148.45 95.888) (end 148.45 94.75) (width 0.2) (layer B.Cu) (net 5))
 (segment (start 148 96.338) (end 148.45 95.888) (width 0.2) (layer B.Cu) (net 5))
 (segment (start 148.4 94.7) (end 148.4 93.5) (width 0.2) (layer B.Cu) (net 5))
 (segment (start 148.45 94.75) (end 148.4 94.7) (width 0.2) (layer B.Cu) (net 5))
 (segment (start 150.7 91) (end 150.81 91) (width 0.2) (layer B.Cu) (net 5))
 (segment (start 148.4 93.3) (end 150.7 91) (width 0.2) (layer B.Cu) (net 5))
 (segment (start 147.1 98.475) (end 147.125 98.5) (width 0.2) (layer B.Cu) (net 5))
 (segment (start 147.65 99.4) (end 147.662 99.35) (width 0.2) (layer B.Cu) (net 5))
 (segment (start 147.65 98.9) (end 147.65 99.4) (width 0.2) (layer B.Cu) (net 5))
 (segment (start 147.25 98.5) (end 147.65 98.9) (width 0.2) (layer B.Cu) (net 5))
 (segment (start 147.125 98.5) (end 147.25 98.5) (width 0.2) (layer B.Cu) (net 5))
 (segment (start 146.85 98.475) (end 147.1 98.475) (width 0.2) (layer B.Cu) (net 5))
 (segment (start 147.1 98.475) (end 147.025 98.475) (width 0.2) (layer B.Cu) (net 5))
 (segment (start 147.1 97.25) (end 147.1 97.238) (width 0.2) (layer B.Cu) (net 5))
 (segment (start 147.1 98.4) (end 147.1 97.25) (width 0.2) (layer B.Cu) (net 5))
 (segment (start 147.025 98.475) (end 147.1 98.4) (width 0.2) (layer B.Cu) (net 5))
 (segment (start 148 96.338) (end 147.1 97.238) (width 0.2) (layer B.Cu) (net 5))
 (segment (start 147.1 97.238) (end 147.1 97.238) (width 0.2) (layer B.Cu) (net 5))
 (segment (start 148 96.338) (end 148.238 96.338) (width 0.2) (layer B.Cu) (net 5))
 (segment (start 149.15 98.35) (end 148.85 98.05) (width 0.2) (layer B.Cu) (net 5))
 (segment (start 148.85 98.05) (end 148.85 96.95) (width 0.2) (layer B.Cu) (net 5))
 (via (at 150.25 98.35) (size 0.5) (layers F.Cu B.Cu) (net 5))
 (segment (start 149.15 98.35) (end 150.25 98.35) (width 0.2) (layer B.Cu) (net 5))
 (segment (start 148.238 96.338) (end 148.85 96.95) (width 0.2) (layer B.Cu) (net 5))
 (segment (start 144.938 97.6) (end 145 97.6) (width 0.2) (layer B.Cu) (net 5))
 (segment (start 145 97.6) (end 145.875 98.475) (width 0.2) (layer B.Cu) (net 5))
 (segment (start 145.875 98.475) (end 146.65 98.475) (width 0.2) (layer B.Cu) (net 5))
 (segment (start 146.65 98.475) (end 146.85 98.475) (width 0.2) (layer B.Cu) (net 5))
 (segment (start 146.85 98.475) (end 146.787 98.475) (width 0.2) (layer B.Cu) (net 5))
 (segment (start 144.938 97.6) (end 144.2 97.6) (width 0.2) (layer B.Cu) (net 5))
 (segment (start 144.2 97.6) (end 143.9 97.3) (width 0.2) (layer B.Cu) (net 5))
 (segment (start 148.95 98.9) (end 150.1 98.9) (width 0.2) (layer F.Cu) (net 5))
 (segment (start 150.15 98.45) (end 150.25 98.35) (width 0.2) (layer F.Cu) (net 5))
 (segment (start 150.15 98.45) (end 148.95 98.45) (width 0.2) (layer F.Cu) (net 5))
 (segment (start 150.25 98.75) (end 150.25 98.35) (width 0.2) (layer F.Cu) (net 5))
 (segment (start 150.1 98.9) (end 150.25 98.75) (width 0.2) (layer F.Cu) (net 5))
 (segment (start 145.05 97.55) (end 144.15 97.55) (width 0.2) (layer F.Cu) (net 5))
 (via (at 143.9 97.3) (size 0.5) (layers F.Cu B.Cu) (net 5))
 (segment (start 144.15 97.55) (end 143.9 97.3) (width 0.2) (layer F.Cu) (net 5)))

